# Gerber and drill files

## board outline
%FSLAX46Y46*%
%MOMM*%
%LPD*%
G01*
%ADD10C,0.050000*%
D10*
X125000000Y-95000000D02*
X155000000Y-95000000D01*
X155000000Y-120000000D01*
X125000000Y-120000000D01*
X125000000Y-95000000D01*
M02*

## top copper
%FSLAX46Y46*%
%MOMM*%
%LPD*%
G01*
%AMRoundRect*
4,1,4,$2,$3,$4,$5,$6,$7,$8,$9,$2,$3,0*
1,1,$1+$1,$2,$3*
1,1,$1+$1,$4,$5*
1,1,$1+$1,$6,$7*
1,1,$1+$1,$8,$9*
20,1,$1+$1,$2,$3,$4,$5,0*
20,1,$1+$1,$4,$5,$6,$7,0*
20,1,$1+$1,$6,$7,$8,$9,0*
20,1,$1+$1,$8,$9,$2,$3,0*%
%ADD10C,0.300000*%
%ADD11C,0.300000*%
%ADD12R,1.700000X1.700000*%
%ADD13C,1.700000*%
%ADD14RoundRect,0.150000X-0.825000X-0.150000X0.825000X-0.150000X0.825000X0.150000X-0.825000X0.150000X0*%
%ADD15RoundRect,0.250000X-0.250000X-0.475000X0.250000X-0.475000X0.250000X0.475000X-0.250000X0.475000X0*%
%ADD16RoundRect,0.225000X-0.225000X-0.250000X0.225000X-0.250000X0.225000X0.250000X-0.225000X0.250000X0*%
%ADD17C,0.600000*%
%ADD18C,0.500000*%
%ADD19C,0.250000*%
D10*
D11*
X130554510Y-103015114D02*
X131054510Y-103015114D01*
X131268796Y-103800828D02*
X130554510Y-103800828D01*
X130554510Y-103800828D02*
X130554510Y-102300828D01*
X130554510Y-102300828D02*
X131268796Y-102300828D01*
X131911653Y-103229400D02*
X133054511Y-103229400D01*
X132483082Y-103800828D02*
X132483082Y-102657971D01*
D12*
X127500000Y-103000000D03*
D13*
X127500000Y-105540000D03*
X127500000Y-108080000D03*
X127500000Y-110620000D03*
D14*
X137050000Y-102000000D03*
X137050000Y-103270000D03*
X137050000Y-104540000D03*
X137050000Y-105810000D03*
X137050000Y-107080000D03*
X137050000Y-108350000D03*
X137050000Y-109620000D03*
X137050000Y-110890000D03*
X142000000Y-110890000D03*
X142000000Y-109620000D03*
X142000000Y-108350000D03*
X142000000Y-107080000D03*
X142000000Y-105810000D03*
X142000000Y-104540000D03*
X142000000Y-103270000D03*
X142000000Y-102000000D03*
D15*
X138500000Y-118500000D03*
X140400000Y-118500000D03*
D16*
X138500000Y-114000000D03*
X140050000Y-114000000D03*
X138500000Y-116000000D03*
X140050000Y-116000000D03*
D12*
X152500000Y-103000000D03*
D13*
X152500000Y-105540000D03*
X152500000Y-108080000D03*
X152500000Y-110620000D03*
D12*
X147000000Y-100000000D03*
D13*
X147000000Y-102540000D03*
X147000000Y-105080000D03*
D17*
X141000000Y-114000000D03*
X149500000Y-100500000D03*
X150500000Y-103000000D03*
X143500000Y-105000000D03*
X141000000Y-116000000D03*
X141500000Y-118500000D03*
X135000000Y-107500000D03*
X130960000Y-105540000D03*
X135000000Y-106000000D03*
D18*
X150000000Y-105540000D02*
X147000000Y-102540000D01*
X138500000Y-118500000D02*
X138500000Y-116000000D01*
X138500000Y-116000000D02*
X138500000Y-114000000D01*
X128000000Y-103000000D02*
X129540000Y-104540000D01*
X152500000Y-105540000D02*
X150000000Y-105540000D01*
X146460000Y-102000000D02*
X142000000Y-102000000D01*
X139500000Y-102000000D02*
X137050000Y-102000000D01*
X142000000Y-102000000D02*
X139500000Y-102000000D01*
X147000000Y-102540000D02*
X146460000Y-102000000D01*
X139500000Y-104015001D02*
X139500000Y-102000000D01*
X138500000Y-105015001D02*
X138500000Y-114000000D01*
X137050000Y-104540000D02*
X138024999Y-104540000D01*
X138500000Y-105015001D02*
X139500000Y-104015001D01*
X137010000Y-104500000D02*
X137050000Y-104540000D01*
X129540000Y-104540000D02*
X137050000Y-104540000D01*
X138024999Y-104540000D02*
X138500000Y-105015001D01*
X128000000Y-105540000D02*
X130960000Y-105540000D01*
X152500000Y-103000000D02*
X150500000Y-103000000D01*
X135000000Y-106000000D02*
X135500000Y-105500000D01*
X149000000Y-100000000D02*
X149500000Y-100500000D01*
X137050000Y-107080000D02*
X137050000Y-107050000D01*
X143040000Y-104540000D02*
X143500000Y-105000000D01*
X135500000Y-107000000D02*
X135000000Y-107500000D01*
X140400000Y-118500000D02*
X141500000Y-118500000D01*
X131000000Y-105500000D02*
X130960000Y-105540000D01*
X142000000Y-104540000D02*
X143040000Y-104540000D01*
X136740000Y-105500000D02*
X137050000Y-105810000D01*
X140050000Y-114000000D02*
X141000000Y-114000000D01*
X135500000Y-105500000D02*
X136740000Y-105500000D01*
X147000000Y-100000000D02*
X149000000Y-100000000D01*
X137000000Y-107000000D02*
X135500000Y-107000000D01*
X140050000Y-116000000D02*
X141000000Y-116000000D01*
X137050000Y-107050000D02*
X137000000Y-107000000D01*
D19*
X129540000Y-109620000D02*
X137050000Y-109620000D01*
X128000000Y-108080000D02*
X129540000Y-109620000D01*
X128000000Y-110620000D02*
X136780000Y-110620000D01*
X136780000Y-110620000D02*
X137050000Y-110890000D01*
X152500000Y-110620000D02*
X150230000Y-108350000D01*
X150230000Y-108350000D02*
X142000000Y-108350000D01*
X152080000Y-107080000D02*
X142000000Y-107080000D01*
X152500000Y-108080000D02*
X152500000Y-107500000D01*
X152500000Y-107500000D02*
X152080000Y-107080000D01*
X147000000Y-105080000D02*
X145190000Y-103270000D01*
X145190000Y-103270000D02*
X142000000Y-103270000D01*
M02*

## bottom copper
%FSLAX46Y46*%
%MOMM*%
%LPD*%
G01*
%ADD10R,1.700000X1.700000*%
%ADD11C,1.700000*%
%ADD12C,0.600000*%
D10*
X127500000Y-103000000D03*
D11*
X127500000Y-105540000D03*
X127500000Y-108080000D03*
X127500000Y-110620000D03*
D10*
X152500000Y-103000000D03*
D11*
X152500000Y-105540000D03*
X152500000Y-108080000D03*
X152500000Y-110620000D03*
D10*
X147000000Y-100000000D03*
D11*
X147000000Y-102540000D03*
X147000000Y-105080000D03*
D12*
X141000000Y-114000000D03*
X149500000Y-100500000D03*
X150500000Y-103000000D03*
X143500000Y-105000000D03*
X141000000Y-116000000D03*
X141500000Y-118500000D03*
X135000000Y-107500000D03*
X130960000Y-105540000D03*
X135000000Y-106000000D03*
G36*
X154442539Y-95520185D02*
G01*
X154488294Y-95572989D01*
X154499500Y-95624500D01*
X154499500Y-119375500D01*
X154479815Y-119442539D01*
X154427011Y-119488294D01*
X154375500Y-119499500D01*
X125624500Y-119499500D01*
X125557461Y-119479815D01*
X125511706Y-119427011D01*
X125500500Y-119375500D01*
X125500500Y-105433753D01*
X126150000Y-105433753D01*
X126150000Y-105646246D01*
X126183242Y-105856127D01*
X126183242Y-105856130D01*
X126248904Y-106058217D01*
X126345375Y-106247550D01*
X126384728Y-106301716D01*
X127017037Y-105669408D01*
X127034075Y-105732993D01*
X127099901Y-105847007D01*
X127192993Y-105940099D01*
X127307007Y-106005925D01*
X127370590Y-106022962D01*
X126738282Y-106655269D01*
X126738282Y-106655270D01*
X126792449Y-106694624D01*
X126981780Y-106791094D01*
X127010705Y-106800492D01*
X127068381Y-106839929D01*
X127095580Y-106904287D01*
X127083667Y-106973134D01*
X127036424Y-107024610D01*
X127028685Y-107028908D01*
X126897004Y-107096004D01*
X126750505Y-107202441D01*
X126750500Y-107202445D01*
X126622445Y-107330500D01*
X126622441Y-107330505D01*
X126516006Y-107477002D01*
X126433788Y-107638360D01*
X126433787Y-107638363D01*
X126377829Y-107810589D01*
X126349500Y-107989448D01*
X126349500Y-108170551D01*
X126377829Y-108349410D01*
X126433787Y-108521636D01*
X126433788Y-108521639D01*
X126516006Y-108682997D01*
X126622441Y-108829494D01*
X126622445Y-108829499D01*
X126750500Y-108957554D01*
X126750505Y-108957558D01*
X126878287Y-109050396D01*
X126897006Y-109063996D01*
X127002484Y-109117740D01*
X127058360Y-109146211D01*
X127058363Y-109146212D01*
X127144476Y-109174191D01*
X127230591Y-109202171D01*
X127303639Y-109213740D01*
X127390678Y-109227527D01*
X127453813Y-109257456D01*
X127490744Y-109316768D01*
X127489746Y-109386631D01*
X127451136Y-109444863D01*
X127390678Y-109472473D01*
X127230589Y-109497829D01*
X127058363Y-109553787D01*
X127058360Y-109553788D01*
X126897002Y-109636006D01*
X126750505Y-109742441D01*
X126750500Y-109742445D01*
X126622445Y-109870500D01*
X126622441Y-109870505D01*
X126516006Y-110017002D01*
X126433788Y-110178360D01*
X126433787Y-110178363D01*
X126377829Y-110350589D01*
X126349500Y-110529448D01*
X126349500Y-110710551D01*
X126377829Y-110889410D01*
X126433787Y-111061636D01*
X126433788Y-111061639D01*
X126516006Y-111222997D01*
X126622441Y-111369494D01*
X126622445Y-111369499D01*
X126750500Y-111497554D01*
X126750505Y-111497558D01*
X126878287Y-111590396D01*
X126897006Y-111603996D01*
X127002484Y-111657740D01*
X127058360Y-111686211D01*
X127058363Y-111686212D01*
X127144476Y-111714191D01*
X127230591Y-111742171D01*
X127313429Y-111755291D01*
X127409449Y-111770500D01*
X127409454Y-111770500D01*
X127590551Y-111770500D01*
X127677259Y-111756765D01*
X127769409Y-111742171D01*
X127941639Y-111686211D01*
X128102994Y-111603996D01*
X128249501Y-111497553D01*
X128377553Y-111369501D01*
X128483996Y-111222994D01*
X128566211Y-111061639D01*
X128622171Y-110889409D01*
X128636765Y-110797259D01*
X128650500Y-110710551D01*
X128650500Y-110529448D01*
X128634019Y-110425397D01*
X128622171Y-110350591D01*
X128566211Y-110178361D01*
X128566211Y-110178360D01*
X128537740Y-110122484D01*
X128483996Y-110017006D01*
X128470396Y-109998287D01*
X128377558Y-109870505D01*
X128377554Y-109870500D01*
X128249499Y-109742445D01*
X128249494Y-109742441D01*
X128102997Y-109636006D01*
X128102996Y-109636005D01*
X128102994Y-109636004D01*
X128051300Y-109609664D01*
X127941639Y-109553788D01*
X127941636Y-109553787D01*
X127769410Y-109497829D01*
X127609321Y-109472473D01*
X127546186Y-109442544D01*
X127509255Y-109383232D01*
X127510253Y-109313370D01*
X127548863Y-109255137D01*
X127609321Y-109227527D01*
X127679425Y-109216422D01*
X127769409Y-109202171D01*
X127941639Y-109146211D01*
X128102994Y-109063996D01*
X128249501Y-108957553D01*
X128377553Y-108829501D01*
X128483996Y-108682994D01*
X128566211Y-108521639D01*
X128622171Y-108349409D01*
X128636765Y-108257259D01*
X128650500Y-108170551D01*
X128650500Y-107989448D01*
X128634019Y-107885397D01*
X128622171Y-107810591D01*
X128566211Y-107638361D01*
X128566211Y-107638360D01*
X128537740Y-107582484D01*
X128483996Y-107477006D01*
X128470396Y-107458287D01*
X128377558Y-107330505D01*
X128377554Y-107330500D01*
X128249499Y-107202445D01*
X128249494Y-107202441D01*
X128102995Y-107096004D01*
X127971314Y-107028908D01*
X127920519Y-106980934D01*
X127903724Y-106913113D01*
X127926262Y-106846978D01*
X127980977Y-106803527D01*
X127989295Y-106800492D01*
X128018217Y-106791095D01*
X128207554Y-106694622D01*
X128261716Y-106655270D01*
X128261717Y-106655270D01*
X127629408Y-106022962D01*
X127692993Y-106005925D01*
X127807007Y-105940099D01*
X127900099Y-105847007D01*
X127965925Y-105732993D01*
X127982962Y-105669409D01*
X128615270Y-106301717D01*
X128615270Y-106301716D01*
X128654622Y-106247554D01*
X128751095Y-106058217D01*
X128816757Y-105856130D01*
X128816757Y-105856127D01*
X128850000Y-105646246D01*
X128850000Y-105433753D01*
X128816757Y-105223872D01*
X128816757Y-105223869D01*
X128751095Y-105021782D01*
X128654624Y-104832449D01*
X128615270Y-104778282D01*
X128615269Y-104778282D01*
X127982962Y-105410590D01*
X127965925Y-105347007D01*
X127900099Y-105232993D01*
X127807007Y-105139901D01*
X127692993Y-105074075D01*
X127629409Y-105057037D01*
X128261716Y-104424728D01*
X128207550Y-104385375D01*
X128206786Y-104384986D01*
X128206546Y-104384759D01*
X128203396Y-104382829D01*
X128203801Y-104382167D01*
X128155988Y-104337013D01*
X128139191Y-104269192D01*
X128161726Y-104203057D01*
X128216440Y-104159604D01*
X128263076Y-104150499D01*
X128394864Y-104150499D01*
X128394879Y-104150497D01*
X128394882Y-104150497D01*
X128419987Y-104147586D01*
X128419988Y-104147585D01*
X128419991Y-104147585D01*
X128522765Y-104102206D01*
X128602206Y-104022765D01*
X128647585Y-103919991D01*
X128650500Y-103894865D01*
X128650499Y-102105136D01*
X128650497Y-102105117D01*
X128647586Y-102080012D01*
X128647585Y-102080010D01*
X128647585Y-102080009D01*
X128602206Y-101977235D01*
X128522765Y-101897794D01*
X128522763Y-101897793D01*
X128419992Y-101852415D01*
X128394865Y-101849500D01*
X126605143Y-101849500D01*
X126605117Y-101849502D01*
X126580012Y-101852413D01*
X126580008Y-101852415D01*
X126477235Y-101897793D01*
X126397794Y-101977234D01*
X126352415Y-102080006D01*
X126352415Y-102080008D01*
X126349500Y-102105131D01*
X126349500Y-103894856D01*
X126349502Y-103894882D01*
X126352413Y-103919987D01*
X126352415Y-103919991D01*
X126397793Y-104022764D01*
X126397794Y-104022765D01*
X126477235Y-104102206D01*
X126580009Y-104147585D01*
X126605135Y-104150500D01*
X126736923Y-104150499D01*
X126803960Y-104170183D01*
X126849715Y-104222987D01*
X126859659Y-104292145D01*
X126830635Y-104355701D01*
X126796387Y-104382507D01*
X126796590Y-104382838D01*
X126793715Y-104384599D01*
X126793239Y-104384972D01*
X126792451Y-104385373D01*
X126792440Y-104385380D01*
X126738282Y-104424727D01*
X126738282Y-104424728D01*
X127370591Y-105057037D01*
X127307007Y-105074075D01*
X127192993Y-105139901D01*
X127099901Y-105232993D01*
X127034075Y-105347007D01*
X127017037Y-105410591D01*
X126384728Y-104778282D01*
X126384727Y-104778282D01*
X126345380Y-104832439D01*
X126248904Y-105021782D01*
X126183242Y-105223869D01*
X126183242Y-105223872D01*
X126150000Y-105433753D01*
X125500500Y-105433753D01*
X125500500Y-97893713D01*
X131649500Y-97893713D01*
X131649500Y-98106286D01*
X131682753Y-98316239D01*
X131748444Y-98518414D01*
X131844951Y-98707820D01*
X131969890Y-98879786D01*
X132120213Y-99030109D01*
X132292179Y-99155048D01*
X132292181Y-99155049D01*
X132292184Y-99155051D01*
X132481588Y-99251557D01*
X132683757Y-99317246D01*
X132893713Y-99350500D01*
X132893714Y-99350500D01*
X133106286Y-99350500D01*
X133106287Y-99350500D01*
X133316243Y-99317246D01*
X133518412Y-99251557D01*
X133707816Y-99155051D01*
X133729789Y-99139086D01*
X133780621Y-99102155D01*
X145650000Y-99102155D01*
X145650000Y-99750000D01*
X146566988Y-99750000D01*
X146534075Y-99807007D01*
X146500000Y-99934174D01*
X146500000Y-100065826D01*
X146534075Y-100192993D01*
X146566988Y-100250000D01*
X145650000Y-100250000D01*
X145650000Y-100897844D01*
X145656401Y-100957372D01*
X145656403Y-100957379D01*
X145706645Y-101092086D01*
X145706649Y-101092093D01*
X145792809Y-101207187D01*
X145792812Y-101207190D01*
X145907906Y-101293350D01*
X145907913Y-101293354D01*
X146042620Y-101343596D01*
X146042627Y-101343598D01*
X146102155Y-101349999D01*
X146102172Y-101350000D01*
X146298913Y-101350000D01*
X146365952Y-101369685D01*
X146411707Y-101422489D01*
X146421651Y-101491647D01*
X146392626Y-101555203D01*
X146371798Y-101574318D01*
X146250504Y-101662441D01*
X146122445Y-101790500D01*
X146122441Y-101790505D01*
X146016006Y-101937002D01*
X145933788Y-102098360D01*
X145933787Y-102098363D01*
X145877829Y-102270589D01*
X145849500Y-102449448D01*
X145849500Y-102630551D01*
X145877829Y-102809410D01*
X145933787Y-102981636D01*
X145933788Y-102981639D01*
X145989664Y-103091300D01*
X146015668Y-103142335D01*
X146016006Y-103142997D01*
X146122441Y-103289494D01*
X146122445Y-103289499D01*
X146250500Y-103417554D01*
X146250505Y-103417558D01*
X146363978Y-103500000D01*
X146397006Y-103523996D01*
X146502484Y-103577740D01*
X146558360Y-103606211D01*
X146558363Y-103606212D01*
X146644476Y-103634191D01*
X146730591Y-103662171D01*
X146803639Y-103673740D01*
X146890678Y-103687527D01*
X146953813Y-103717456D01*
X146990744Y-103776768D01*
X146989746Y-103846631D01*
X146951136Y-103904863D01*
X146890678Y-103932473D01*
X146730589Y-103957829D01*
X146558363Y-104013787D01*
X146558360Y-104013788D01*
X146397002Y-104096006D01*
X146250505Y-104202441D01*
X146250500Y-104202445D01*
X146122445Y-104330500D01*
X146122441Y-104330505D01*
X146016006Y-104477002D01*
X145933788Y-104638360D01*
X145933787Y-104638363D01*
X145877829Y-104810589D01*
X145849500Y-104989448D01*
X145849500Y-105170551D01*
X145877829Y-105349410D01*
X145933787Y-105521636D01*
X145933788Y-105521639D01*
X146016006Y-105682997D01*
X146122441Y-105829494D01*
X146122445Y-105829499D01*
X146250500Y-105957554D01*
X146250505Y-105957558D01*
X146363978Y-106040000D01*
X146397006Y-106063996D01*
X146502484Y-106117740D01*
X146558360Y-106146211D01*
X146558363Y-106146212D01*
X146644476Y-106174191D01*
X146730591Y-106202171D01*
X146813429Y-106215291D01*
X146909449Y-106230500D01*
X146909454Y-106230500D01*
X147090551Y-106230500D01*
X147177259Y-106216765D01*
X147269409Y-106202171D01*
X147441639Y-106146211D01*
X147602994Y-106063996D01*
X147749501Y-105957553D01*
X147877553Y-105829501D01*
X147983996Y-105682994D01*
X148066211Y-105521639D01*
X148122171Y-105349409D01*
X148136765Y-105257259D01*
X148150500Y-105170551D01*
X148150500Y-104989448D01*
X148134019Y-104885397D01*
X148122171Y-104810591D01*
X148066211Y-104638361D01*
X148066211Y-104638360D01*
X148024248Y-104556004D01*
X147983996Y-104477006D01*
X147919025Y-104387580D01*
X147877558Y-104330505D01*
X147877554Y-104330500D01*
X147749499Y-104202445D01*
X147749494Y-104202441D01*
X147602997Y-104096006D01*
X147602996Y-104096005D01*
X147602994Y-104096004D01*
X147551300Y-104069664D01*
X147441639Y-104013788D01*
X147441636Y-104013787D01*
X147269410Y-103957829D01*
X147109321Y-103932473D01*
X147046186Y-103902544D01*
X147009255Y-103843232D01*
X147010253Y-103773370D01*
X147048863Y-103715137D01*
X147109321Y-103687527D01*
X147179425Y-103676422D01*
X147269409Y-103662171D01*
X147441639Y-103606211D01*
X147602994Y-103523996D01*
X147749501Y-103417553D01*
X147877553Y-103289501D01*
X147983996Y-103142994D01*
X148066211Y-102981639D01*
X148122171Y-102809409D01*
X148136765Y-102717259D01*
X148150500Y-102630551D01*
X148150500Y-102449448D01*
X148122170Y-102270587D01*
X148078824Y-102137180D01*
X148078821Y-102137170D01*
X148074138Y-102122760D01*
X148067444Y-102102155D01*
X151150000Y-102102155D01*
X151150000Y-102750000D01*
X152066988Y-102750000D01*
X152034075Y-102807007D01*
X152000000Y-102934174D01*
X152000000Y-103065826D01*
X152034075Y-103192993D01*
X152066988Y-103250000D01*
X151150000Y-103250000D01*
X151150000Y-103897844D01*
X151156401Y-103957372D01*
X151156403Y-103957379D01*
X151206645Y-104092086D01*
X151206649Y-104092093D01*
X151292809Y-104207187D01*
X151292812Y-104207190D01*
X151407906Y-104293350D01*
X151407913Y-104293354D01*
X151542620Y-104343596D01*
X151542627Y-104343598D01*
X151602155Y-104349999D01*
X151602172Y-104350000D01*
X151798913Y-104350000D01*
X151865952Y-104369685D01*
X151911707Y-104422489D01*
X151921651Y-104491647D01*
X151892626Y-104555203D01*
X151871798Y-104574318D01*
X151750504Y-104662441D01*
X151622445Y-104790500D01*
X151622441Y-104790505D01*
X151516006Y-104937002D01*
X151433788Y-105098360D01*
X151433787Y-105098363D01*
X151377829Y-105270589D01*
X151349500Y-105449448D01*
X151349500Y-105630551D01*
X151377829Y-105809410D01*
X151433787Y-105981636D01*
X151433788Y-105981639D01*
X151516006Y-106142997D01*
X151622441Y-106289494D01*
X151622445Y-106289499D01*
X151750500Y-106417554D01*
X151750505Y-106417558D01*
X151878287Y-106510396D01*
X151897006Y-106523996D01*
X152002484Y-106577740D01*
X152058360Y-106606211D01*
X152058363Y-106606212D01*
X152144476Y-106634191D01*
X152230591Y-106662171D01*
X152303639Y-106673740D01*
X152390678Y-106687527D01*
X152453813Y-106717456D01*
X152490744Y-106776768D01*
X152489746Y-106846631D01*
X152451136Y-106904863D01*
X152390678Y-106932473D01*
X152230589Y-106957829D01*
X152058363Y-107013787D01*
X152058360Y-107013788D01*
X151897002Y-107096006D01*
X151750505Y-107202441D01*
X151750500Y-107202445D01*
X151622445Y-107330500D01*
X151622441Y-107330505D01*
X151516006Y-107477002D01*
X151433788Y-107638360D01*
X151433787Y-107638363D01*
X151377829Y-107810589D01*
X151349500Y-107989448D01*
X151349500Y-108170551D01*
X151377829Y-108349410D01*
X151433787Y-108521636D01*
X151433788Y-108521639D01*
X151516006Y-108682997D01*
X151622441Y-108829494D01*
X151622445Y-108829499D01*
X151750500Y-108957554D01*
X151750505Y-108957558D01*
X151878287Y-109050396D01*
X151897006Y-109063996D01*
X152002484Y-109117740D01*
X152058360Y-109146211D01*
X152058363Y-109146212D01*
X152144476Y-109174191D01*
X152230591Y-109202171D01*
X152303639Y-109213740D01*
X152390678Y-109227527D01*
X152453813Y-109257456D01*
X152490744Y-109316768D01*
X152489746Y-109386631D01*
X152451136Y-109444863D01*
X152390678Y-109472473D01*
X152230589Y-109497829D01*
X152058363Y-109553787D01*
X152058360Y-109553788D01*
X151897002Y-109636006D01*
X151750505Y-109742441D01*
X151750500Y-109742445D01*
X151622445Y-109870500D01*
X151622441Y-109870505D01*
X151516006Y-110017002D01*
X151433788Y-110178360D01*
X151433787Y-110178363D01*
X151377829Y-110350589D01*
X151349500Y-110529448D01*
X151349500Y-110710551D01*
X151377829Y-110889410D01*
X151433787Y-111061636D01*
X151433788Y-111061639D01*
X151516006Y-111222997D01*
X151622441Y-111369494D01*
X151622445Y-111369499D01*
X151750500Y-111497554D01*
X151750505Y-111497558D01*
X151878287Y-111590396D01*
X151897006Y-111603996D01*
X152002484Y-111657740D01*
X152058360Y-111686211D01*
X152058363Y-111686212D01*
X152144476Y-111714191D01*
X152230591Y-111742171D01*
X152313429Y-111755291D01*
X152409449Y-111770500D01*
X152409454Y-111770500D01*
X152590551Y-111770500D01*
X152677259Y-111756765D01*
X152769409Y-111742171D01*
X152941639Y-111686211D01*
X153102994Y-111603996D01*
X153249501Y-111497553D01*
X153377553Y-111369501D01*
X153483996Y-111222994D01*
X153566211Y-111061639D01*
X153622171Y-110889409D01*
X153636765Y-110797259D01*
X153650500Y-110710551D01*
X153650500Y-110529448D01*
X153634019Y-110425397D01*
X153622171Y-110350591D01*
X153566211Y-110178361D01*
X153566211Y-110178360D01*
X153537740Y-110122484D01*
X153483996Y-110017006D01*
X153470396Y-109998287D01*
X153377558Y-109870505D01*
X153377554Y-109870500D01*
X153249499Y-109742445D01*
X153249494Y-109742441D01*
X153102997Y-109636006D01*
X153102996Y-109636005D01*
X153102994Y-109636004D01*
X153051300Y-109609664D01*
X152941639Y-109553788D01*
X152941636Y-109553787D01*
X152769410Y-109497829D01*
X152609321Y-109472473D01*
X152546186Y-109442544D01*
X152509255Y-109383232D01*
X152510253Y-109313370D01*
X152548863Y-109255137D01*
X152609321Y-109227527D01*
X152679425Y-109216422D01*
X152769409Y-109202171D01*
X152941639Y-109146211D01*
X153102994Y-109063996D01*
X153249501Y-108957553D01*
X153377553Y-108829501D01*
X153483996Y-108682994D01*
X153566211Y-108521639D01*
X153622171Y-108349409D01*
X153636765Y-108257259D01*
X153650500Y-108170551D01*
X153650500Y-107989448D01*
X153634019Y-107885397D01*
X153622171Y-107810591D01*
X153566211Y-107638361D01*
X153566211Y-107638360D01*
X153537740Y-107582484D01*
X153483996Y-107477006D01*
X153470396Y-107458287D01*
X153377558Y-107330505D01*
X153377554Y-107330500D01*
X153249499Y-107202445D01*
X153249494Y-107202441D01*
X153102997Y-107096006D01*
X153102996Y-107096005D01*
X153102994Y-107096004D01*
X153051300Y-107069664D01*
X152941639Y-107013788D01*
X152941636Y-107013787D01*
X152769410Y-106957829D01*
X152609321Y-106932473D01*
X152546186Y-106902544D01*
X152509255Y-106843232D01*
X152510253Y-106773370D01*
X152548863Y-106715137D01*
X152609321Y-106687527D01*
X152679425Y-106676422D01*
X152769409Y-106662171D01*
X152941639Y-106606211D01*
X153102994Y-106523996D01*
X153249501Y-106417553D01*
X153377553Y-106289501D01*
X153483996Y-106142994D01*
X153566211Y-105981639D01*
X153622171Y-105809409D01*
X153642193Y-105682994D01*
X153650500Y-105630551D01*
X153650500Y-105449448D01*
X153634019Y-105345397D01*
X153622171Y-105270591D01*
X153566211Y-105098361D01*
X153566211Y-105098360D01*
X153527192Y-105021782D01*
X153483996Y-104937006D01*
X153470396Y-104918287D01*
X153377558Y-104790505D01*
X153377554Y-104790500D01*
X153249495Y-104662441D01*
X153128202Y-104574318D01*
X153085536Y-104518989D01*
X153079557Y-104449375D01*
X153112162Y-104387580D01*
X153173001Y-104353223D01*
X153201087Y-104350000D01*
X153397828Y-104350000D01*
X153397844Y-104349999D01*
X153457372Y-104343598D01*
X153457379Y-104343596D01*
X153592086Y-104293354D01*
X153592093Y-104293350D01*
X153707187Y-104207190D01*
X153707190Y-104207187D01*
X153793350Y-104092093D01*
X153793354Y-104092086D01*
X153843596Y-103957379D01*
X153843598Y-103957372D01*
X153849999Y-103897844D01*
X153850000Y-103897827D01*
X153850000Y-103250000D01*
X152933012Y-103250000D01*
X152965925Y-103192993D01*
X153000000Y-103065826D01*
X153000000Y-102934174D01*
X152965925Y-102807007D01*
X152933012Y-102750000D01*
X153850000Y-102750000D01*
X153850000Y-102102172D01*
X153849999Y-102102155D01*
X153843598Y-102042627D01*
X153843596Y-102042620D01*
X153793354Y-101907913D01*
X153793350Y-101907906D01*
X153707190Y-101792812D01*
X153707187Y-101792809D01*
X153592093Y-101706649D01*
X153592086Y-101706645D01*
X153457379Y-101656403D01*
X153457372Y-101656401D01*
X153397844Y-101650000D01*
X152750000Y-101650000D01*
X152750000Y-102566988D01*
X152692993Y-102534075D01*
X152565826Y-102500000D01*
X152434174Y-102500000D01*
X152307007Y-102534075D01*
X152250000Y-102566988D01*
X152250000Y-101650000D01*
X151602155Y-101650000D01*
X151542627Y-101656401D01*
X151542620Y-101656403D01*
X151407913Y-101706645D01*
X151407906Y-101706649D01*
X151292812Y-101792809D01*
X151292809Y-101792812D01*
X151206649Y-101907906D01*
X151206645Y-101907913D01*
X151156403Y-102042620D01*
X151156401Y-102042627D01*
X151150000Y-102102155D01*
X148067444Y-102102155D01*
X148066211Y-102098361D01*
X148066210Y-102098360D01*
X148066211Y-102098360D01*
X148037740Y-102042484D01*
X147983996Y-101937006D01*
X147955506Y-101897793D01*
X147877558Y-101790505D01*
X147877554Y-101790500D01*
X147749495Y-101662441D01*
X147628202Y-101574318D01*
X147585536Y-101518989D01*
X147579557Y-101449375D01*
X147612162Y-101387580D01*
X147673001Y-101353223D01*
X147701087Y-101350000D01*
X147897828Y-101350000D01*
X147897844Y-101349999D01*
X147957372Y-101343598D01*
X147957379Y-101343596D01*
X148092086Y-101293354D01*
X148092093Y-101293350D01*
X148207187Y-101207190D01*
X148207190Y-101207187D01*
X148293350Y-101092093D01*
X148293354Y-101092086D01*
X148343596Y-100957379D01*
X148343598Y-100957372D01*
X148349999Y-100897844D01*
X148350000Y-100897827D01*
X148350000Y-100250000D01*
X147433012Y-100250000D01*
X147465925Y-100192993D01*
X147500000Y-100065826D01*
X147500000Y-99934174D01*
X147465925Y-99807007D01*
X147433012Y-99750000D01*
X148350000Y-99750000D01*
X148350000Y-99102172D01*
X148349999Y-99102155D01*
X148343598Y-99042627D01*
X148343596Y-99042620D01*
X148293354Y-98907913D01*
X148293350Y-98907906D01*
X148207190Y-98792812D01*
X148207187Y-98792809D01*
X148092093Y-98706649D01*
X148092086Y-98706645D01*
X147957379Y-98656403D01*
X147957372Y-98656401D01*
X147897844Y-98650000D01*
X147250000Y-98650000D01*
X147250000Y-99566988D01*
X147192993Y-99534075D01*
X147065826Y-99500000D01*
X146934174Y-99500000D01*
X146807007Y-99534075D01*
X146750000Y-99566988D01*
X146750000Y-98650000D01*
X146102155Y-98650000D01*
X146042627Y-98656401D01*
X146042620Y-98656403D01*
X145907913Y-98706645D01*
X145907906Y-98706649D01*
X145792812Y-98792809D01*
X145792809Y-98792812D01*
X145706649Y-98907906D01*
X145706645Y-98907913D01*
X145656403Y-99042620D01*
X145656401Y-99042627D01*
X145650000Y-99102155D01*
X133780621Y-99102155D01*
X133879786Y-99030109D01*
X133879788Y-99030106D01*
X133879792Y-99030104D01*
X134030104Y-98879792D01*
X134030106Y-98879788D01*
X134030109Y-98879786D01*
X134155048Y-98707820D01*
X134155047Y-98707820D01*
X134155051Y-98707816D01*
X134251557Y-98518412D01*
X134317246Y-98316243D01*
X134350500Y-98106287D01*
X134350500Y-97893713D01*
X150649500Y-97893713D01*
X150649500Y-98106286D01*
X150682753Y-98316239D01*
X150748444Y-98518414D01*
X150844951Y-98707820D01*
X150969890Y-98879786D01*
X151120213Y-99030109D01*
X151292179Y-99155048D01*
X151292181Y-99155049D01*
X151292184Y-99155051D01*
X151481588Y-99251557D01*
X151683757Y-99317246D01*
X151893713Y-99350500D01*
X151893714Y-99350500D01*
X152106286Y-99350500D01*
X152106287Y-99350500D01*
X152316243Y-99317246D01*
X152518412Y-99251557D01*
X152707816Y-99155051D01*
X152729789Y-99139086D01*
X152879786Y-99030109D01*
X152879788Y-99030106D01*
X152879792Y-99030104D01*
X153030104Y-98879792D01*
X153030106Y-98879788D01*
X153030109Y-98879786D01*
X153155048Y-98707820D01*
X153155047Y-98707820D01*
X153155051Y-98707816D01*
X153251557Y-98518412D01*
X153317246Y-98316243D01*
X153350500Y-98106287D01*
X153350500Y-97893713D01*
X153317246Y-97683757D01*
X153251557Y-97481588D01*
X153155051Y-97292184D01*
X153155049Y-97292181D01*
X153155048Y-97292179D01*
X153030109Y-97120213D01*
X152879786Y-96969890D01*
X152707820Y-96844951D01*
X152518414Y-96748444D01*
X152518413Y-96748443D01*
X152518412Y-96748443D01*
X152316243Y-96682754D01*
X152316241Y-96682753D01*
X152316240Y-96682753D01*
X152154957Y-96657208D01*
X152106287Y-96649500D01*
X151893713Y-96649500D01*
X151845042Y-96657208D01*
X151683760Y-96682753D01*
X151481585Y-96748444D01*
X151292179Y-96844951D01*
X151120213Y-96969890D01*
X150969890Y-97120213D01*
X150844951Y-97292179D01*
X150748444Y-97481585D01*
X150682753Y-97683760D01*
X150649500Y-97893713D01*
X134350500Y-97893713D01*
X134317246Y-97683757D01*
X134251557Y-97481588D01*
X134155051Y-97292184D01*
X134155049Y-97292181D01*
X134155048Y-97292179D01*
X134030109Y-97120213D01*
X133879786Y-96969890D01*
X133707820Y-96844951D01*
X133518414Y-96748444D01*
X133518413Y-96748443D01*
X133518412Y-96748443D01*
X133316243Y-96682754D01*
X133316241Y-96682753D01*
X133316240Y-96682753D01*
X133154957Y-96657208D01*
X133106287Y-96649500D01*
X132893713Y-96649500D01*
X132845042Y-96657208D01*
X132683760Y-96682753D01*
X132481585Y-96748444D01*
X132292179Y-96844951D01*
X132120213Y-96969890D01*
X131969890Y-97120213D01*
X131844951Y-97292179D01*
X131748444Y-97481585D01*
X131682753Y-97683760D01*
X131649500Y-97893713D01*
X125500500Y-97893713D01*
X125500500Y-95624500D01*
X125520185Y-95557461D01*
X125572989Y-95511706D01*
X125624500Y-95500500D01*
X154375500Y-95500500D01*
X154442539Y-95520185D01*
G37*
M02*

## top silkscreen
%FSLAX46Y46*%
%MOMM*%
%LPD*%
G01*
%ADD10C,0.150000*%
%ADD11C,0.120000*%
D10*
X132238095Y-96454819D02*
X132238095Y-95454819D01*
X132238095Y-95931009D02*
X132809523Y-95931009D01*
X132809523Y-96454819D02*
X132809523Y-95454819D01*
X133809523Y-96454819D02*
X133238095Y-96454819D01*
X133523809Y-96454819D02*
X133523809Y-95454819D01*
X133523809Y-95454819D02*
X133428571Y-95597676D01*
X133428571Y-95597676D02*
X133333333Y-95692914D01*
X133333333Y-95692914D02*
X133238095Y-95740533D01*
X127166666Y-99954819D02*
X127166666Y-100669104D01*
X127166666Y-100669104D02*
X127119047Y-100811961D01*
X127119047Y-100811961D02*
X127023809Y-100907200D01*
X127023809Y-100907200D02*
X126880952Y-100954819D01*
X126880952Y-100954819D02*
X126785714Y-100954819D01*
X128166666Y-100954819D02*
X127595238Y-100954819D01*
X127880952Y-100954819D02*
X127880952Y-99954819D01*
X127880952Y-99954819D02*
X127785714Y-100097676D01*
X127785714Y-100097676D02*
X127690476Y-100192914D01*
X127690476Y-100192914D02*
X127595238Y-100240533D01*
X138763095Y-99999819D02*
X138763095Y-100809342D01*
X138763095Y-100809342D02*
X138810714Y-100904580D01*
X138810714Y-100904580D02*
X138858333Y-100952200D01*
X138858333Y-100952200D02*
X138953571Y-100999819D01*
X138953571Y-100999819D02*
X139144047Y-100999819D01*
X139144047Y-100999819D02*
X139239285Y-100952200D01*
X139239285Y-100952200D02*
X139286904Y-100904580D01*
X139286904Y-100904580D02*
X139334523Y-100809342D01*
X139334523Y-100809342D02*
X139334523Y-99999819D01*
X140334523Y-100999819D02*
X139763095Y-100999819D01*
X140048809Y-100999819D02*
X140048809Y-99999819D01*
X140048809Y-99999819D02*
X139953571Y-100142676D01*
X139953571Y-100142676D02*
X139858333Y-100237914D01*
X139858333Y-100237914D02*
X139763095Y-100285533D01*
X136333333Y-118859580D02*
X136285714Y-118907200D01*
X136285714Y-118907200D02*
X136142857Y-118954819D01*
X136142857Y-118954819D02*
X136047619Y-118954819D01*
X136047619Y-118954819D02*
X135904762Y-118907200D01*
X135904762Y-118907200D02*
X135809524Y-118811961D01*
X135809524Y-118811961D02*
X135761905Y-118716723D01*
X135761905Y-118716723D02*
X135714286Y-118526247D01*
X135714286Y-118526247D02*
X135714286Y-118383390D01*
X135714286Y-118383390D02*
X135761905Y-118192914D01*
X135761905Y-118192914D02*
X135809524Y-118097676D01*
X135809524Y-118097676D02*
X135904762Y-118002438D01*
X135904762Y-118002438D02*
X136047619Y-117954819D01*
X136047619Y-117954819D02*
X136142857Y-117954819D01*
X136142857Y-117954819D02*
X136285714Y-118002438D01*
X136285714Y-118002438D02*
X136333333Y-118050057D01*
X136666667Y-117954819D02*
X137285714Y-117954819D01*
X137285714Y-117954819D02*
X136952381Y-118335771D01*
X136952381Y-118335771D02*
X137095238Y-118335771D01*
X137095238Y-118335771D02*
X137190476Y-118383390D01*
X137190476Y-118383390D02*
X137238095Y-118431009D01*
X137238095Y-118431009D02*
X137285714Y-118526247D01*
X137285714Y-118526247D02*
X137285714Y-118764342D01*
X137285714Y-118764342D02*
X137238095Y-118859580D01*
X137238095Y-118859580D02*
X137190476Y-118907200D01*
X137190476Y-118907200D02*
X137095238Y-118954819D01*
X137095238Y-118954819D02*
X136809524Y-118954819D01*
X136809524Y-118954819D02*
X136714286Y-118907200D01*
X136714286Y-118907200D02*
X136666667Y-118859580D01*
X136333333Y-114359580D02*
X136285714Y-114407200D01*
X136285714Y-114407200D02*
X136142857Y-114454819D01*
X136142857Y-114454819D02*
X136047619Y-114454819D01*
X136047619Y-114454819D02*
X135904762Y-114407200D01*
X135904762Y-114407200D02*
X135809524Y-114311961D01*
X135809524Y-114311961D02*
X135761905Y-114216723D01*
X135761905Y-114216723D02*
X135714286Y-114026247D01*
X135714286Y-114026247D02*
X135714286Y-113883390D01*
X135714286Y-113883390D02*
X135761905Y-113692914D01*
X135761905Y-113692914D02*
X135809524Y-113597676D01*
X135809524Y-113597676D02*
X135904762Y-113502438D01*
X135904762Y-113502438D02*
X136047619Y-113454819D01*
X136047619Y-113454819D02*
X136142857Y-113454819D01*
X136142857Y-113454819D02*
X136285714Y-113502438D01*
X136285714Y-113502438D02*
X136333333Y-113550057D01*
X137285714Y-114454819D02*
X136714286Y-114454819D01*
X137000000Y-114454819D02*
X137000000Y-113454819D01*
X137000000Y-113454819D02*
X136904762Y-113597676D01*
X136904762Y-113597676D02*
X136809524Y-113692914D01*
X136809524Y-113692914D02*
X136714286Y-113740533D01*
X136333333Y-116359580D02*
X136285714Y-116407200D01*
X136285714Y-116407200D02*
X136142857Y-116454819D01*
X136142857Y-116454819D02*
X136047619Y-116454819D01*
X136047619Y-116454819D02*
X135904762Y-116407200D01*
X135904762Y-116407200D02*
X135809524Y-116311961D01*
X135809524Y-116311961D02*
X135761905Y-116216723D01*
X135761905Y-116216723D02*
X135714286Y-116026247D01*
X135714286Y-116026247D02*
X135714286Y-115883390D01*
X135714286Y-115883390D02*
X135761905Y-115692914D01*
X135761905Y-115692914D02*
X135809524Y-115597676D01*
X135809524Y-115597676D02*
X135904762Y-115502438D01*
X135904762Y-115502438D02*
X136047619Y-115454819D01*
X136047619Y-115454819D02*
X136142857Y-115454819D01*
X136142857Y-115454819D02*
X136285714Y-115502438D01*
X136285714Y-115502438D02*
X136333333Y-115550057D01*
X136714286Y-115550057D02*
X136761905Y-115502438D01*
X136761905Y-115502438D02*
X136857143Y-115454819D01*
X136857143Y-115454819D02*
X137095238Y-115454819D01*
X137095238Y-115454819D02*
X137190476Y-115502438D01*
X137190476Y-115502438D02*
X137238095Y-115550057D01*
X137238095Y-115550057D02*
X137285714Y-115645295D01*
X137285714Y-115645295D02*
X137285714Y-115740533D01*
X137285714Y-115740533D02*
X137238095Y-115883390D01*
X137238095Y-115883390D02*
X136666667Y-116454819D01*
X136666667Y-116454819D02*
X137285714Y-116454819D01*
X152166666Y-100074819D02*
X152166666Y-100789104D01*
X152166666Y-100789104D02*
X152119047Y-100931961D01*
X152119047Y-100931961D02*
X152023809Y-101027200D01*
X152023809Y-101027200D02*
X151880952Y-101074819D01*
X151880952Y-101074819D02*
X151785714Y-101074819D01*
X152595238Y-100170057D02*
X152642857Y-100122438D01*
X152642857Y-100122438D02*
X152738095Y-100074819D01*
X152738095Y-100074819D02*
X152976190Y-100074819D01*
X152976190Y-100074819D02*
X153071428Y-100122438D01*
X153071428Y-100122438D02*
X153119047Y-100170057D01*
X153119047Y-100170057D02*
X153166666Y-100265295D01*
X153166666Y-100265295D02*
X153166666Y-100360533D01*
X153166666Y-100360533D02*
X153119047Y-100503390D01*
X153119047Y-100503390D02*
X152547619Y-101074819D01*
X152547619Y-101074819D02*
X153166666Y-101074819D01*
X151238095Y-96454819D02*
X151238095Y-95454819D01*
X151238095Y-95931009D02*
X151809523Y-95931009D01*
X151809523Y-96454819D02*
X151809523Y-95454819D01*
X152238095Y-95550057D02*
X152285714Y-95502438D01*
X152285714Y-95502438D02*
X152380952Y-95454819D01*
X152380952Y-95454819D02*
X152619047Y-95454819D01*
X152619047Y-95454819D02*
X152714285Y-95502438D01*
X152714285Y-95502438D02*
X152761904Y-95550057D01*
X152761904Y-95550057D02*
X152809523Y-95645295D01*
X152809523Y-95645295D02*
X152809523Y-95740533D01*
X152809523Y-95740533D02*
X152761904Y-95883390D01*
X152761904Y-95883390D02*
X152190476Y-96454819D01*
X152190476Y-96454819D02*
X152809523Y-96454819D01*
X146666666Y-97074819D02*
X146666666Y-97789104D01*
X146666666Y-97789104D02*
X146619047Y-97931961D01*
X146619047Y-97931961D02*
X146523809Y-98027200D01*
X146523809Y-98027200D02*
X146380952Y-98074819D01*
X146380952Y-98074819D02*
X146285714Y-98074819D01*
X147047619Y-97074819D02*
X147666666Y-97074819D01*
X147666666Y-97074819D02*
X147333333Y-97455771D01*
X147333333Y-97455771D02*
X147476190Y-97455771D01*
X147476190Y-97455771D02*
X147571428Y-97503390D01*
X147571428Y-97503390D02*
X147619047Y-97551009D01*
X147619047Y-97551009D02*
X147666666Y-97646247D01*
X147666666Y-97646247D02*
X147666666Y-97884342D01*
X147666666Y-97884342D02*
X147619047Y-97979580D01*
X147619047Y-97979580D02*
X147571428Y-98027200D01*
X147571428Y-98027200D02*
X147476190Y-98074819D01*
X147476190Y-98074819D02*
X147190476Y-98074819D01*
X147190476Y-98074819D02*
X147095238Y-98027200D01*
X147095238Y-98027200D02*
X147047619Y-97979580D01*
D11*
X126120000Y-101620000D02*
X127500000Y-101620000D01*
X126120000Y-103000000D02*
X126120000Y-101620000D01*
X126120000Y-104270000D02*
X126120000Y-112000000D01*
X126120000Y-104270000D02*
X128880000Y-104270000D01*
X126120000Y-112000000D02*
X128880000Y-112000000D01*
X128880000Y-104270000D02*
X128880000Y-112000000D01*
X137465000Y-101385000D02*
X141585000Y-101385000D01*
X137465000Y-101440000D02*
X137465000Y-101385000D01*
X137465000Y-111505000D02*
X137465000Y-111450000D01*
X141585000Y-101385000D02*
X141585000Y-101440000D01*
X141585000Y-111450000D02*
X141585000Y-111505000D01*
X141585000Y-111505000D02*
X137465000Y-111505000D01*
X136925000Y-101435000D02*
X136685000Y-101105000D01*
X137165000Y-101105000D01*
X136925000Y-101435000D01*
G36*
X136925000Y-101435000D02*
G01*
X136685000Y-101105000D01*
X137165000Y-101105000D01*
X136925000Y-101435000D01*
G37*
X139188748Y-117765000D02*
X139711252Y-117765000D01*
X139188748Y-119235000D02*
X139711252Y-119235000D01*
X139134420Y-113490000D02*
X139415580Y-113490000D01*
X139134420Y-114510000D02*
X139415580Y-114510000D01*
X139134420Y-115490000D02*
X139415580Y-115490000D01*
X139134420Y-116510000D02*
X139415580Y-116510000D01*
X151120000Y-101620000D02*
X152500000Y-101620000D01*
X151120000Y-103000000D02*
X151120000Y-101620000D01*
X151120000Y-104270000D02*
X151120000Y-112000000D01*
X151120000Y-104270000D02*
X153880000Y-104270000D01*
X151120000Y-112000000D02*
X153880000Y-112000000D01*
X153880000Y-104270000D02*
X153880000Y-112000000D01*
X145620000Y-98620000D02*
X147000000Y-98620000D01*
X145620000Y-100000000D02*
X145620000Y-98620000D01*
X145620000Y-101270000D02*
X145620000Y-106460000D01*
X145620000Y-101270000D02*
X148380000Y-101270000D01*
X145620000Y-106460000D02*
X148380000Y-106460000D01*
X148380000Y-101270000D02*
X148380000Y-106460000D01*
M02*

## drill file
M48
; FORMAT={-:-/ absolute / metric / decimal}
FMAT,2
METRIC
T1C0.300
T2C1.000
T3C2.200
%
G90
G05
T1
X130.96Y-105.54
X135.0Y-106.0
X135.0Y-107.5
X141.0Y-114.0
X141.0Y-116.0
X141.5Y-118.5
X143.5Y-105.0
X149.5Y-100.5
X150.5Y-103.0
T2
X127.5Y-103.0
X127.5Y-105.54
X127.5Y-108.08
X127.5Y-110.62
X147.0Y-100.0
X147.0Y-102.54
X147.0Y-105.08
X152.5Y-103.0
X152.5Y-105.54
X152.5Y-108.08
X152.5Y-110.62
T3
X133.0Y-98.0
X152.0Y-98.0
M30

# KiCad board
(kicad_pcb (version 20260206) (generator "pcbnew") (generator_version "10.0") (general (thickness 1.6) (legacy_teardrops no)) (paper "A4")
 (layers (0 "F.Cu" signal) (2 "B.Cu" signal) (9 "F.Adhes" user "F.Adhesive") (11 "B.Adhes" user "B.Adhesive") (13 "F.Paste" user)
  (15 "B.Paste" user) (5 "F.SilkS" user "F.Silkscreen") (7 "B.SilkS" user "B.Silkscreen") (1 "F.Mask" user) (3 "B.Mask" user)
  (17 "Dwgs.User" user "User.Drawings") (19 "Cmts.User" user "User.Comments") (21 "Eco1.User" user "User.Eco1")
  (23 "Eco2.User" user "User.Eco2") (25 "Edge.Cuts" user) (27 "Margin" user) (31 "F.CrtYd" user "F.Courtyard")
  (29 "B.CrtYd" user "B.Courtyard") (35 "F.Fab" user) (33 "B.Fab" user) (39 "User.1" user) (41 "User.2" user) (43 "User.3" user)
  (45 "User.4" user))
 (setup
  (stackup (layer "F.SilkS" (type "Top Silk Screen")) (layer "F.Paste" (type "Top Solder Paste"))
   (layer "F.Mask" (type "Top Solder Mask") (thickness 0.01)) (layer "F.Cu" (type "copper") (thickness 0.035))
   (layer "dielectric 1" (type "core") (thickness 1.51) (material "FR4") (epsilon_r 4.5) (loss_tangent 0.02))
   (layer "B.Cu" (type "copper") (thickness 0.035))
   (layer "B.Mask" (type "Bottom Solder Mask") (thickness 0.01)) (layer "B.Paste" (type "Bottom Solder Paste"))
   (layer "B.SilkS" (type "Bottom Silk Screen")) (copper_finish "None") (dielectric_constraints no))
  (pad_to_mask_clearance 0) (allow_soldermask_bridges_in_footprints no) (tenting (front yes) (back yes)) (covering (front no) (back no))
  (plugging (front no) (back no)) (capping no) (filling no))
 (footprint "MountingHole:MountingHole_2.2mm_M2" (layer "F.Cu") (at 133 98)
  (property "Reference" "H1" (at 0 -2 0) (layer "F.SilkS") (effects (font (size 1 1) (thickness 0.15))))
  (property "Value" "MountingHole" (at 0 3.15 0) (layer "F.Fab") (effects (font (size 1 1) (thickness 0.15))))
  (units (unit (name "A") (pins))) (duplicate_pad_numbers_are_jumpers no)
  (pad "" np_thru_hole circle (at 0 0) (size 2.2 2.2) (drill 2.2) (layers "*.Cu" "*.Mask")))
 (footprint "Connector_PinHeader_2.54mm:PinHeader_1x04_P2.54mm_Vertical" (layer "F.Cu") (at 127.5 103)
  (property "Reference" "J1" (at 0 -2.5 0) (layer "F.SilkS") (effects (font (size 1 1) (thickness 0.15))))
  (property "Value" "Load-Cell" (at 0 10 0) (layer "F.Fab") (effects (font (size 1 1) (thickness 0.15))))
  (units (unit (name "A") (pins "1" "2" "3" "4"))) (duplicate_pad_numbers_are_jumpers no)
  (fp_line (start -1.38 -1.38) (end 0 -1.38) (stroke (width 0.12) (type solid)) (layer "F.SilkS"))
  (fp_line (start -1.38 0) (end -1.38 -1.38) (stroke (width 0.12) (type solid)) (layer "F.SilkS"))
  (fp_line (start -1.38 1.27) (end -1.38 9) (stroke (width 0.12) (type solid)) (layer "F.SilkS"))
  (fp_line (start -1.38 1.27) (end 1.38 1.27) (stroke (width 0.12) (type solid)) (layer "F.SilkS"))
  (fp_line (start -1.38 9) (end 1.38 9) (stroke (width 0.12) (type solid)) (layer "F.SilkS"))
  (fp_line (start 1.38 1.27) (end 1.38 9) (stroke (width 0.12) (type solid)) (layer "F.SilkS"))
  (pad "1" thru_hole rect (at 0 0) (size 1.7 1.7) (drill 1) (layers "*.Cu" "*.Mask") (remove_unused_layers no) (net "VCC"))
  (pad "2" thru_hole circle (at 0 2.54) (size 1.7 1.7) (drill 1) (layers "*.Cu" "*.Mask") (remove_unused_layers no) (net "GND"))
  (pad "3" thru_hole circle (at 0 5.08) (size 1.7 1.7) (drill 1) (layers "*.Cu" "*.Mask") (remove_unused_layers no) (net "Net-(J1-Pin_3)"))
  (pad "4" thru_hole circle (at 0 7.62) (size 1.7 1.7) (drill 1) (layers "*.Cu" "*.Mask") (remove_unused_layers no) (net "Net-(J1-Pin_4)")))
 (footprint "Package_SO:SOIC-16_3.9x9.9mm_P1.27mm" (layer "F.Cu") (at 139.525 106.445)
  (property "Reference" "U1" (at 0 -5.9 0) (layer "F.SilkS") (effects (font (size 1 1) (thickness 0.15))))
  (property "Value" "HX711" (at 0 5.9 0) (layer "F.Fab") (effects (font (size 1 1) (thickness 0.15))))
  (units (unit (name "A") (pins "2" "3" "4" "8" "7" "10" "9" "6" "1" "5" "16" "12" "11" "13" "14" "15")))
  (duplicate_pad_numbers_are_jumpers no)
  (fp_line (start -2.06 -5.06) (end 2.06 -5.06) (stroke (width 0.12) (type solid)) (layer "F.SilkS"))
  (fp_line (start -2.06 -5.005) (end -2.06 -5.06) (stroke (width 0.12) (type solid)) (layer "F.SilkS"))
  (fp_line (start -2.06 5.06) (end -2.06 5.005) (stroke (width 0.12) (type solid)) (layer "F.SilkS"))
  (fp_line (start 2.06 -5.06) (end 2.06 -5.005) (stroke (width 0.12) (type solid)) (layer "F.SilkS"))
  (fp_line (start 2.06 5.005) (end 2.06 5.06) (stroke (width 0.12) (type solid)) (layer "F.SilkS"))
  (fp_line (start 2.06 5.06) (end -2.06 5.06) (stroke (width 0.12) (type solid)) (layer "F.SilkS"))
  (fp_poly (pts (xy -2.6 -5.01) (xy -2.84 -5.34) (xy -2.36 -5.34)) (stroke (width 0.12) (type solid)) (fill yes) (layer "F.SilkS"))
  (pad "1" smd roundrect (at -2.475 -4.445) (size 1.95 0.6) (layers "F.Cu" "F.Mask" "F.Paste") (roundrect_rratio 0.25) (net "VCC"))
  (pad "2" smd roundrect (at -2.475 -3.175) (size 1.95 0.6) (layers "F.Cu" "F.Mask" "F.Paste") (roundrect_rratio 0.25)
   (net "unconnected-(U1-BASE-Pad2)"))
  (pad "3" smd roundrect (at -2.475 -1.905) (size 1.95 0.6) (layers "F.Cu" "F.Mask" "F.Paste") (roundrect_rratio 0.25) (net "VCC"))
  (pad "4" smd roundrect (at -2.475 -0.635) (size 1.95 0.6) (layers "F.Cu" "F.Mask" "F.Paste") (roundrect_rratio 0.25) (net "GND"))
  (pad "5" smd roundrect (at -2.475 0.635) (size 1.95 0.6) (layers "F.Cu" "F.Mask" "F.Paste") (roundrect_rratio 0.25) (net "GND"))
  (pad "6" smd roundrect (at -2.475 1.905) (size 1.95 0.6) (layers "F.Cu" "F.Mask" "F.Paste") (roundrect_rratio 0.25)
   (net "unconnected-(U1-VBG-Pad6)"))
  (pad "7" smd roundrect (at -2.475 3.175) (size 1.95 0.6) (layers "F.Cu" "F.Mask" "F.Paste") (roundrect_rratio 0.25) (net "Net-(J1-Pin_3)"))
  (pad "8" smd roundrect (at -2.475 4.445) (size 1.95 0.6) (layers "F.Cu" "F.Mask" "F.Paste") (roundrect_rratio 0.25) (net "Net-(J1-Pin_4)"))
  (pad "9" smd roundrect (at 2.475 4.445) (size 1.95 0.6) (layers "F.Cu" "F.Mask" "F.Paste") (roundrect_rratio 0.25)
   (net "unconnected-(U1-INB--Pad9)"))
  (pad "10" smd roundrect (at 2.475 3.175) (size 1.95 0.6) (layers "F.Cu" "F.Mask" "F.Paste") (roundrect_rratio 0.25)
   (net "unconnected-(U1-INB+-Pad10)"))
  (pad "11" smd roundrect (at 2.475 1.905) (size 1.95 0.6) (layers "F.Cu" "F.Mask" "F.Paste") (roundrect_rratio 0.25) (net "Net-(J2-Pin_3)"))
  (pad "12" smd roundrect (at 2.475 0.635) (size 1.95 0.6) (layers "F.Cu" "F.Mask" "F.Paste") (roundrect_rratio 0.25) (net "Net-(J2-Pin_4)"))
  (pad "13" smd roundrect (at 2.475 -0.635) (size 1.95 0.6) (layers "F.Cu" "F.Mask" "F.Paste") (roundrect_rratio 0.25)
   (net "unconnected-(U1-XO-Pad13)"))
  (pad "14" smd roundrect (at 2.475 -1.905) (size 1.95 0.6) (layers "F.Cu" "F.Mask" "F.Paste") (roundrect_rratio 0.25) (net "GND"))
  (pad "15" smd roundrect (at 2.475 -3.175) (size 1.95 0.6) (layers "F.Cu" "F.Mask" "F.Paste") (roundrect_rratio 0.25) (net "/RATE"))
  (pad "16" smd roundrect (at 2.475 -4.445) (size 1.95 0.6) (layers "F.Cu" "F.Mask" "F.Paste") (roundrect_rratio 0.25) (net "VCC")))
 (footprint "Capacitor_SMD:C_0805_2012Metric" (layer "F.Cu") (at 139.45 118.5)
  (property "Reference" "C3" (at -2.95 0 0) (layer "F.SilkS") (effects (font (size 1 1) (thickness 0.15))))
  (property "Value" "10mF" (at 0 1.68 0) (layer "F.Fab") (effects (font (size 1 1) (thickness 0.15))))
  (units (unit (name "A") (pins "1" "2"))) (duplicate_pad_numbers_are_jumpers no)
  (fp_line (start -0.261252 -0.735) (end 0.261252 -0.735) (stroke (width 0.12) (type solid)) (layer "F.SilkS"))
  (fp_line (start -0.261252 0.735) (end 0.261252 0.735) (stroke (width 0.12) (type solid)) (layer "F.SilkS"))
  (pad "1" smd roundrect (at -0.95 0) (size 1 1.45) (layers "F.Cu" "F.Mask" "F.Paste") (roundrect_rratio 0.25) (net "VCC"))
  (pad "2" smd roundrect (at 0.95 0) (size 1 1.45) (layers "F.Cu" "F.Mask" "F.Paste") (roundrect_rratio 0.25) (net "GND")))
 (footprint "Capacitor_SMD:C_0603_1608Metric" (layer "F.Cu") (at 139.275 114)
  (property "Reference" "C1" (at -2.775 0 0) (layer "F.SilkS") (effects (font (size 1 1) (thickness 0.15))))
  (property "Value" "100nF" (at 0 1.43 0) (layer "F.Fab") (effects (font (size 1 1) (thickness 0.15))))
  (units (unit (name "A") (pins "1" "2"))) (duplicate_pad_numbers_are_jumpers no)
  (fp_line (start -0.14058 -0.51) (end 0.14058 -0.51) (stroke (width 0.12) (type solid)) (layer "F.SilkS"))
  (fp_line (start -0.14058 0.51) (end 0.14058 0.51) (stroke (width 0.12) (type solid)) (layer "F.SilkS"))
  (pad "1" smd roundrect (at -0.775 0) (size 0.9 0.95) (layers "F.Cu" "F.Mask" "F.Paste") (roundrect_rratio 0.25) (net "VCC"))
  (pad "2" smd roundrect (at 0.775 0) (size 0.9 0.95) (layers "F.Cu" "F.Mask" "F.Paste") (roundrect_rratio 0.25) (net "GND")))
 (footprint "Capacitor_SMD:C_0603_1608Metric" (layer "F.Cu") (at 139.275 116)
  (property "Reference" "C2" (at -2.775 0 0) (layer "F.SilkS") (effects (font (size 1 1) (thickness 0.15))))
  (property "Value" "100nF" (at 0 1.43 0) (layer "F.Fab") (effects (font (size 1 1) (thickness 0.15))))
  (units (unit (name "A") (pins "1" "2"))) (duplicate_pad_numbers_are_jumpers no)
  (fp_line (start -0.14058 -0.51) (end 0.14058 -0.51) (stroke (width 0.12) (type solid)) (layer "F.SilkS"))
  (fp_line (start -0.14058 0.51) (end 0.14058 0.51) (stroke (width 0.12) (type solid)) (layer "F.SilkS"))
  (pad "1" smd roundrect (at -0.775 0) (size 0.9 0.95) (layers "F.Cu" "F.Mask" "F.Paste") (roundrect_rratio 0.25) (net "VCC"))
  (pad "2" smd roundrect (at 0.775 0) (size 0.9 0.95) (layers "F.Cu" "F.Mask" "F.Paste") (roundrect_rratio 0.25) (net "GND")))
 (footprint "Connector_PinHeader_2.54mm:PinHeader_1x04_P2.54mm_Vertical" (layer "F.Cu") (at 152.5 103)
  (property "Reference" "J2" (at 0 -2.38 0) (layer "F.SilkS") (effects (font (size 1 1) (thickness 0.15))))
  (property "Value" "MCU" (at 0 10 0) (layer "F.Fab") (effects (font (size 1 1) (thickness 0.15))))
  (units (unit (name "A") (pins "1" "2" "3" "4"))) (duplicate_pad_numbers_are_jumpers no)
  (fp_line (start -1.38 -1.38) (end 0 -1.38) (stroke (width 0.12) (type solid)) (layer "F.SilkS"))
  (fp_line (start -1.38 0) (end -1.38 -1.38) (stroke (width 0.12) (type solid)) (layer "F.SilkS"))
  (fp_line (start -1.38 1.27) (end -1.38 9) (stroke (width 0.12) (type solid)) (layer "F.SilkS"))
  (fp_line (start -1.38 1.27) (end 1.38 1.27) (stroke (width 0.12) (type solid)) (layer "F.SilkS"))
  (fp_line (start -1.38 9) (end 1.38 9) (stroke (width 0.12) (type solid)) (layer "F.SilkS"))
  (fp_line (start 1.38 1.27) (end 1.38 9) (stroke (width 0.12) (type solid)) (layer "F.SilkS"))
  (pad "1" thru_hole rect (at 0 0) (size 1.7 1.7) (drill 1) (layers "*.Cu" "*.Mask") (remove_unused_layers no) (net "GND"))
  (pad "2" thru_hole circle (at 0 2.54) (size 1.7 1.7) (drill 1) (layers "*.Cu" "*.Mask") (remove_unused_layers no) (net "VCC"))
  (pad "3" thru_hole circle (at 0 5.08) (size 1.7 1.7) (drill 1) (layers "*.Cu" "*.Mask") (remove_unused_layers no) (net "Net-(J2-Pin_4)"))
  (pad "4" thru_hole circle (at 0 7.62) (size 1.7 1.7) (drill 1) (layers "*.Cu" "*.Mask") (remove_unused_layers no) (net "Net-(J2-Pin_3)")))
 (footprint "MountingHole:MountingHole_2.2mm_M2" (layer "F.Cu") (at 152 98)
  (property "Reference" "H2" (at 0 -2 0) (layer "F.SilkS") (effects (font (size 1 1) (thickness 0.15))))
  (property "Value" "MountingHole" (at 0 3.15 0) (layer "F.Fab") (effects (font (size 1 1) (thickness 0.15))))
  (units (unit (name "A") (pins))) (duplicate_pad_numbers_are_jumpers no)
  (pad "" np_thru_hole circle (at 0 0) (size 2.2 2.2) (drill 2.2) (layers "*.Cu" "*.Mask")))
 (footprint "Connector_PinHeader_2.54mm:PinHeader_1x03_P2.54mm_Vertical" (layer "F.Cu") (at 147 100)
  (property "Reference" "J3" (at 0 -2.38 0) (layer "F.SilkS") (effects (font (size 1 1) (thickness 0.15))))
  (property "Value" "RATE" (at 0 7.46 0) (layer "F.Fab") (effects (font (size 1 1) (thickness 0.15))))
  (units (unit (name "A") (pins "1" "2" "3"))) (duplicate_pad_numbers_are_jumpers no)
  (fp_line (start -1.38 -1.38) (end 0 -1.38) (stroke (width 0.12) (type solid)) (layer "F.SilkS"))
  (fp_line (start -1.38 0) (end -1.38 -1.38) (stroke (width 0.12) (type solid)) (layer "F.SilkS"))
  (fp_line (start -1.38 1.27) (end -1.38 6.46) (stroke (width 0.12) (type solid)) (layer "F.SilkS"))
  (fp_line (start -1.38 1.27) (end 1.38 1.27) (stroke (width 0.12) (type solid)) (layer "F.SilkS"))
  (fp_line (start -1.38 6.46) (end 1.38 6.46) (stroke (width 0.12) (type solid)) (layer "F.SilkS"))
  (fp_line (start 1.38 1.27) (end 1.38 6.46) (stroke (width 0.12) (type solid)) (layer "F.SilkS"))
  (pad "1" thru_hole rect (at 0 0) (size 1.7 1.7) (drill 1) (layers "*.Cu" "*.Mask") (remove_unused_layers no) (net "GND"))
  (pad "2" thru_hole circle (at 0 2.54) (size 1.7 1.7) (drill 1) (layers "*.Cu" "*.Mask") (remove_unused_layers no) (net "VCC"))
  (pad "3" thru_hole circle (at 0 5.08) (size 1.7 1.7) (drill 1) (layers "*.Cu" "*.Mask") (remove_unused_layers no) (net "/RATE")))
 (gr_rect (start 125 95) (end 155 120) (stroke (width 0.05) (type default)) (fill no) (layer "Edge.Cuts"))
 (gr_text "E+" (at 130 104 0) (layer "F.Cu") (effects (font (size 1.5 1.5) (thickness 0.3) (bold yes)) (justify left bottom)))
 (segment (start 150 105.54) (end 147 102.54) (width 0.5) (layer "F.Cu") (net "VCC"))
 (segment (start 138.5 118.5) (end 138.5 116) (width 0.5) (layer "F.Cu") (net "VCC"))
 (segment (start 138.5 116) (end 138.5 114) (width 0.5) (layer "F.Cu") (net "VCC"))
 (segment (start 128 103) (end 129.54 104.54) (width 0.5) (layer "F.Cu") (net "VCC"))
 (segment (start 152.5 105.54) (end 150 105.54) (width 0.5) (layer "F.Cu") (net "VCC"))
 (segment (start 146.46 102) (end 142 102) (width 0.5) (layer "F.Cu") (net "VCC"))
 (segment (start 139.5 102) (end 137.05 102) (width 0.5) (layer "F.Cu") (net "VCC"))
 (segment (start 142 102) (end 139.5 102) (width 0.5) (layer "F.Cu") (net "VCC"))
 (segment (start 147 102.54) (end 146.46 102) (width 0.5) (layer "F.Cu") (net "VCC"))
 (segment (start 139.5 104.015001) (end 139.5 102) (width 0.5) (layer "F.Cu") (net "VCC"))
 (segment (start 138.5 105.015001) (end 138.5 114) (width 0.5) (layer "F.Cu") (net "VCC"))
 (segment (start 137.05 104.54) (end 138.024999 104.54) (width 0.5) (layer "F.Cu") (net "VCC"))
 (segment (start 138.5 105.015001) (end 139.5 104.015001) (width 0.5) (layer "F.Cu") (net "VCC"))
 (segment (start 137.01 104.5) (end 137.05 104.54) (width 0.5) (layer "F.Cu") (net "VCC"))
 (segment (start 129.54 104.54) (end 137.05 104.54) (width 0.5) (layer "F.Cu") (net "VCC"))
 (segment (start 138.024999 104.54) (end 138.5 105.015001) (width 0.5) (layer "F.Cu") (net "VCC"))
 (segment (start 128 105.54) (end 130.96 105.54) (width 0.5) (layer "F.Cu") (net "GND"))
 (segment (start 152.5 103) (end 150.5 103) (width 0.5) (layer "F.Cu") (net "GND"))
 (segment (start 135 106) (end 135.5 105.5) (width 0.5) (layer "F.Cu") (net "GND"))
 (segment (start 149 100) (end 149.5 100.5) (width 0.5) (layer "F.Cu") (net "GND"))
 (segment (start 137.05 107.08) (end 137.05 107.05) (width 0.5) (layer "F.Cu") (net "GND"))
 (segment (start 143.04 104.54) (end 143.5 105) (width 0.5) (layer "F.Cu") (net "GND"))
 (segment (start 135.5 107) (end 135 107.5) (width 0.5) (layer "F.Cu") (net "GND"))
 (segment (start 140.4 118.5) (end 141.5 118.5) (width 0.5) (layer "F.Cu") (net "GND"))
 (segment (start 131 105.5) (end 130.96 105.54) (width 0.5) (layer "F.Cu") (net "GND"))
 (segment (start 142 104.54) (end 143.04 104.54) (width 0.5) (layer "F.Cu") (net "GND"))
 (segment (start 136.74 105.5) (end 137.05 105.81) (width 0.5) (layer "F.Cu") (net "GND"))
 (segment (start 140.05 114) (end 141 114) (width 0.5) (layer "F.Cu") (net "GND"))
 (segment (start 135.5 105.5) (end 136.74 105.5) (width 0.5) (layer "F.Cu") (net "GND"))
 (segment (start 147 100) (end 149 100) (width 0.5) (layer "F.Cu") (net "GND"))
 (segment (start 137 107) (end 135.5 107) (width 0.5) (layer "F.Cu") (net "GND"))
 (segment (start 140.05 116) (end 141 116) (width 0.5) (layer "F.Cu") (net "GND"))
 (segment (start 137.05 107.05) (end 137 107) (width 0.5) (layer "F.Cu") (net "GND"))
 (via (at 141 114) (size 0.6) (drill 0.3) (layers "F.Cu" "B.Cu") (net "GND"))
 (via (at 149.5 100.5) (size 0.6) (drill 0.3) (layers "F.Cu" "B.Cu") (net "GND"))
 (via (at 150.5 103) (size 0.6) (drill 0.3) (layers "F.Cu" "B.Cu") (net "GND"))
 (via (at 143.5 105) (size 0.6) (drill 0.3) (layers "F.Cu" "B.Cu") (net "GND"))
 (via (at 141 116) (size 0.6) (drill 0.3) (layers "F.Cu" "B.Cu") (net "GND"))
 (via (at 141.5 118.5) (size 0.6) (drill 0.3) (layers "F.Cu" "B.Cu") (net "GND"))
 (via (at 135 107.5) (size 0.6) (drill 0.3) (layers "F.Cu" "B.Cu") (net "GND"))
 (via (at 130.96 105.54) (size 0.6) (drill 0.3) (layers "F.Cu" "B.Cu") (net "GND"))
 (via (at 135 106) (size 0.6) (drill 0.3) (layers "F.Cu" "B.Cu") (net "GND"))
 (segment (start 129.54 109.62) (end 137.05 109.62) (width 0.25) (layer "F.Cu") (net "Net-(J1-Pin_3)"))
 (segment (start 128 108.08) (end 129.54 109.62) (width 0.25) (layer "F.Cu") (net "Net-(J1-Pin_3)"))
 (segment (start 128 110.62) (end 136.78 110.62) (width 0.25) (layer "F.Cu") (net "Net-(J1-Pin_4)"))
 (segment (start 136.78 110.62) (end 137.05 110.89) (width 0.25) (layer "F.Cu") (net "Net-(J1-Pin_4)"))
 (segment (start 152.5 110.62) (end 150.23 108.35) (width 0.25) (layer "F.Cu") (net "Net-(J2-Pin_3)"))
 (segment (start 150.23 108.35) (end 142 108.35) (width 0.25) (layer "F.Cu") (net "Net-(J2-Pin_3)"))
 (segment (start 152.08 107.08) (end 142 107.08) (width 0.25) (layer "F.Cu") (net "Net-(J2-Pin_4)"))
 (segment (start 152.5 108.08) (end 152.5 107.5) (width 0.25) (layer "F.Cu") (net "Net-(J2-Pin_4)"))
 (segment (start 152.5 107.5) (end 152.08 107.08) (width 0.25) (layer "F.Cu") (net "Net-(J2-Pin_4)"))
 (segment (start 147 105.08) (end 145.19 103.27) (width 0.25) (layer "F.Cu") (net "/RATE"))
 (segment (start 145.19 103.27) (end 142 103.27) (width 0.25) (layer "F.Cu") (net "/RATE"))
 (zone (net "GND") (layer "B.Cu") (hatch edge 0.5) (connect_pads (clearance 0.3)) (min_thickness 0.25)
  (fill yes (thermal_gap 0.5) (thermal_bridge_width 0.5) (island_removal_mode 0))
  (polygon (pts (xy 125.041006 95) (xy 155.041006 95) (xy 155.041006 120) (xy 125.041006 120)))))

